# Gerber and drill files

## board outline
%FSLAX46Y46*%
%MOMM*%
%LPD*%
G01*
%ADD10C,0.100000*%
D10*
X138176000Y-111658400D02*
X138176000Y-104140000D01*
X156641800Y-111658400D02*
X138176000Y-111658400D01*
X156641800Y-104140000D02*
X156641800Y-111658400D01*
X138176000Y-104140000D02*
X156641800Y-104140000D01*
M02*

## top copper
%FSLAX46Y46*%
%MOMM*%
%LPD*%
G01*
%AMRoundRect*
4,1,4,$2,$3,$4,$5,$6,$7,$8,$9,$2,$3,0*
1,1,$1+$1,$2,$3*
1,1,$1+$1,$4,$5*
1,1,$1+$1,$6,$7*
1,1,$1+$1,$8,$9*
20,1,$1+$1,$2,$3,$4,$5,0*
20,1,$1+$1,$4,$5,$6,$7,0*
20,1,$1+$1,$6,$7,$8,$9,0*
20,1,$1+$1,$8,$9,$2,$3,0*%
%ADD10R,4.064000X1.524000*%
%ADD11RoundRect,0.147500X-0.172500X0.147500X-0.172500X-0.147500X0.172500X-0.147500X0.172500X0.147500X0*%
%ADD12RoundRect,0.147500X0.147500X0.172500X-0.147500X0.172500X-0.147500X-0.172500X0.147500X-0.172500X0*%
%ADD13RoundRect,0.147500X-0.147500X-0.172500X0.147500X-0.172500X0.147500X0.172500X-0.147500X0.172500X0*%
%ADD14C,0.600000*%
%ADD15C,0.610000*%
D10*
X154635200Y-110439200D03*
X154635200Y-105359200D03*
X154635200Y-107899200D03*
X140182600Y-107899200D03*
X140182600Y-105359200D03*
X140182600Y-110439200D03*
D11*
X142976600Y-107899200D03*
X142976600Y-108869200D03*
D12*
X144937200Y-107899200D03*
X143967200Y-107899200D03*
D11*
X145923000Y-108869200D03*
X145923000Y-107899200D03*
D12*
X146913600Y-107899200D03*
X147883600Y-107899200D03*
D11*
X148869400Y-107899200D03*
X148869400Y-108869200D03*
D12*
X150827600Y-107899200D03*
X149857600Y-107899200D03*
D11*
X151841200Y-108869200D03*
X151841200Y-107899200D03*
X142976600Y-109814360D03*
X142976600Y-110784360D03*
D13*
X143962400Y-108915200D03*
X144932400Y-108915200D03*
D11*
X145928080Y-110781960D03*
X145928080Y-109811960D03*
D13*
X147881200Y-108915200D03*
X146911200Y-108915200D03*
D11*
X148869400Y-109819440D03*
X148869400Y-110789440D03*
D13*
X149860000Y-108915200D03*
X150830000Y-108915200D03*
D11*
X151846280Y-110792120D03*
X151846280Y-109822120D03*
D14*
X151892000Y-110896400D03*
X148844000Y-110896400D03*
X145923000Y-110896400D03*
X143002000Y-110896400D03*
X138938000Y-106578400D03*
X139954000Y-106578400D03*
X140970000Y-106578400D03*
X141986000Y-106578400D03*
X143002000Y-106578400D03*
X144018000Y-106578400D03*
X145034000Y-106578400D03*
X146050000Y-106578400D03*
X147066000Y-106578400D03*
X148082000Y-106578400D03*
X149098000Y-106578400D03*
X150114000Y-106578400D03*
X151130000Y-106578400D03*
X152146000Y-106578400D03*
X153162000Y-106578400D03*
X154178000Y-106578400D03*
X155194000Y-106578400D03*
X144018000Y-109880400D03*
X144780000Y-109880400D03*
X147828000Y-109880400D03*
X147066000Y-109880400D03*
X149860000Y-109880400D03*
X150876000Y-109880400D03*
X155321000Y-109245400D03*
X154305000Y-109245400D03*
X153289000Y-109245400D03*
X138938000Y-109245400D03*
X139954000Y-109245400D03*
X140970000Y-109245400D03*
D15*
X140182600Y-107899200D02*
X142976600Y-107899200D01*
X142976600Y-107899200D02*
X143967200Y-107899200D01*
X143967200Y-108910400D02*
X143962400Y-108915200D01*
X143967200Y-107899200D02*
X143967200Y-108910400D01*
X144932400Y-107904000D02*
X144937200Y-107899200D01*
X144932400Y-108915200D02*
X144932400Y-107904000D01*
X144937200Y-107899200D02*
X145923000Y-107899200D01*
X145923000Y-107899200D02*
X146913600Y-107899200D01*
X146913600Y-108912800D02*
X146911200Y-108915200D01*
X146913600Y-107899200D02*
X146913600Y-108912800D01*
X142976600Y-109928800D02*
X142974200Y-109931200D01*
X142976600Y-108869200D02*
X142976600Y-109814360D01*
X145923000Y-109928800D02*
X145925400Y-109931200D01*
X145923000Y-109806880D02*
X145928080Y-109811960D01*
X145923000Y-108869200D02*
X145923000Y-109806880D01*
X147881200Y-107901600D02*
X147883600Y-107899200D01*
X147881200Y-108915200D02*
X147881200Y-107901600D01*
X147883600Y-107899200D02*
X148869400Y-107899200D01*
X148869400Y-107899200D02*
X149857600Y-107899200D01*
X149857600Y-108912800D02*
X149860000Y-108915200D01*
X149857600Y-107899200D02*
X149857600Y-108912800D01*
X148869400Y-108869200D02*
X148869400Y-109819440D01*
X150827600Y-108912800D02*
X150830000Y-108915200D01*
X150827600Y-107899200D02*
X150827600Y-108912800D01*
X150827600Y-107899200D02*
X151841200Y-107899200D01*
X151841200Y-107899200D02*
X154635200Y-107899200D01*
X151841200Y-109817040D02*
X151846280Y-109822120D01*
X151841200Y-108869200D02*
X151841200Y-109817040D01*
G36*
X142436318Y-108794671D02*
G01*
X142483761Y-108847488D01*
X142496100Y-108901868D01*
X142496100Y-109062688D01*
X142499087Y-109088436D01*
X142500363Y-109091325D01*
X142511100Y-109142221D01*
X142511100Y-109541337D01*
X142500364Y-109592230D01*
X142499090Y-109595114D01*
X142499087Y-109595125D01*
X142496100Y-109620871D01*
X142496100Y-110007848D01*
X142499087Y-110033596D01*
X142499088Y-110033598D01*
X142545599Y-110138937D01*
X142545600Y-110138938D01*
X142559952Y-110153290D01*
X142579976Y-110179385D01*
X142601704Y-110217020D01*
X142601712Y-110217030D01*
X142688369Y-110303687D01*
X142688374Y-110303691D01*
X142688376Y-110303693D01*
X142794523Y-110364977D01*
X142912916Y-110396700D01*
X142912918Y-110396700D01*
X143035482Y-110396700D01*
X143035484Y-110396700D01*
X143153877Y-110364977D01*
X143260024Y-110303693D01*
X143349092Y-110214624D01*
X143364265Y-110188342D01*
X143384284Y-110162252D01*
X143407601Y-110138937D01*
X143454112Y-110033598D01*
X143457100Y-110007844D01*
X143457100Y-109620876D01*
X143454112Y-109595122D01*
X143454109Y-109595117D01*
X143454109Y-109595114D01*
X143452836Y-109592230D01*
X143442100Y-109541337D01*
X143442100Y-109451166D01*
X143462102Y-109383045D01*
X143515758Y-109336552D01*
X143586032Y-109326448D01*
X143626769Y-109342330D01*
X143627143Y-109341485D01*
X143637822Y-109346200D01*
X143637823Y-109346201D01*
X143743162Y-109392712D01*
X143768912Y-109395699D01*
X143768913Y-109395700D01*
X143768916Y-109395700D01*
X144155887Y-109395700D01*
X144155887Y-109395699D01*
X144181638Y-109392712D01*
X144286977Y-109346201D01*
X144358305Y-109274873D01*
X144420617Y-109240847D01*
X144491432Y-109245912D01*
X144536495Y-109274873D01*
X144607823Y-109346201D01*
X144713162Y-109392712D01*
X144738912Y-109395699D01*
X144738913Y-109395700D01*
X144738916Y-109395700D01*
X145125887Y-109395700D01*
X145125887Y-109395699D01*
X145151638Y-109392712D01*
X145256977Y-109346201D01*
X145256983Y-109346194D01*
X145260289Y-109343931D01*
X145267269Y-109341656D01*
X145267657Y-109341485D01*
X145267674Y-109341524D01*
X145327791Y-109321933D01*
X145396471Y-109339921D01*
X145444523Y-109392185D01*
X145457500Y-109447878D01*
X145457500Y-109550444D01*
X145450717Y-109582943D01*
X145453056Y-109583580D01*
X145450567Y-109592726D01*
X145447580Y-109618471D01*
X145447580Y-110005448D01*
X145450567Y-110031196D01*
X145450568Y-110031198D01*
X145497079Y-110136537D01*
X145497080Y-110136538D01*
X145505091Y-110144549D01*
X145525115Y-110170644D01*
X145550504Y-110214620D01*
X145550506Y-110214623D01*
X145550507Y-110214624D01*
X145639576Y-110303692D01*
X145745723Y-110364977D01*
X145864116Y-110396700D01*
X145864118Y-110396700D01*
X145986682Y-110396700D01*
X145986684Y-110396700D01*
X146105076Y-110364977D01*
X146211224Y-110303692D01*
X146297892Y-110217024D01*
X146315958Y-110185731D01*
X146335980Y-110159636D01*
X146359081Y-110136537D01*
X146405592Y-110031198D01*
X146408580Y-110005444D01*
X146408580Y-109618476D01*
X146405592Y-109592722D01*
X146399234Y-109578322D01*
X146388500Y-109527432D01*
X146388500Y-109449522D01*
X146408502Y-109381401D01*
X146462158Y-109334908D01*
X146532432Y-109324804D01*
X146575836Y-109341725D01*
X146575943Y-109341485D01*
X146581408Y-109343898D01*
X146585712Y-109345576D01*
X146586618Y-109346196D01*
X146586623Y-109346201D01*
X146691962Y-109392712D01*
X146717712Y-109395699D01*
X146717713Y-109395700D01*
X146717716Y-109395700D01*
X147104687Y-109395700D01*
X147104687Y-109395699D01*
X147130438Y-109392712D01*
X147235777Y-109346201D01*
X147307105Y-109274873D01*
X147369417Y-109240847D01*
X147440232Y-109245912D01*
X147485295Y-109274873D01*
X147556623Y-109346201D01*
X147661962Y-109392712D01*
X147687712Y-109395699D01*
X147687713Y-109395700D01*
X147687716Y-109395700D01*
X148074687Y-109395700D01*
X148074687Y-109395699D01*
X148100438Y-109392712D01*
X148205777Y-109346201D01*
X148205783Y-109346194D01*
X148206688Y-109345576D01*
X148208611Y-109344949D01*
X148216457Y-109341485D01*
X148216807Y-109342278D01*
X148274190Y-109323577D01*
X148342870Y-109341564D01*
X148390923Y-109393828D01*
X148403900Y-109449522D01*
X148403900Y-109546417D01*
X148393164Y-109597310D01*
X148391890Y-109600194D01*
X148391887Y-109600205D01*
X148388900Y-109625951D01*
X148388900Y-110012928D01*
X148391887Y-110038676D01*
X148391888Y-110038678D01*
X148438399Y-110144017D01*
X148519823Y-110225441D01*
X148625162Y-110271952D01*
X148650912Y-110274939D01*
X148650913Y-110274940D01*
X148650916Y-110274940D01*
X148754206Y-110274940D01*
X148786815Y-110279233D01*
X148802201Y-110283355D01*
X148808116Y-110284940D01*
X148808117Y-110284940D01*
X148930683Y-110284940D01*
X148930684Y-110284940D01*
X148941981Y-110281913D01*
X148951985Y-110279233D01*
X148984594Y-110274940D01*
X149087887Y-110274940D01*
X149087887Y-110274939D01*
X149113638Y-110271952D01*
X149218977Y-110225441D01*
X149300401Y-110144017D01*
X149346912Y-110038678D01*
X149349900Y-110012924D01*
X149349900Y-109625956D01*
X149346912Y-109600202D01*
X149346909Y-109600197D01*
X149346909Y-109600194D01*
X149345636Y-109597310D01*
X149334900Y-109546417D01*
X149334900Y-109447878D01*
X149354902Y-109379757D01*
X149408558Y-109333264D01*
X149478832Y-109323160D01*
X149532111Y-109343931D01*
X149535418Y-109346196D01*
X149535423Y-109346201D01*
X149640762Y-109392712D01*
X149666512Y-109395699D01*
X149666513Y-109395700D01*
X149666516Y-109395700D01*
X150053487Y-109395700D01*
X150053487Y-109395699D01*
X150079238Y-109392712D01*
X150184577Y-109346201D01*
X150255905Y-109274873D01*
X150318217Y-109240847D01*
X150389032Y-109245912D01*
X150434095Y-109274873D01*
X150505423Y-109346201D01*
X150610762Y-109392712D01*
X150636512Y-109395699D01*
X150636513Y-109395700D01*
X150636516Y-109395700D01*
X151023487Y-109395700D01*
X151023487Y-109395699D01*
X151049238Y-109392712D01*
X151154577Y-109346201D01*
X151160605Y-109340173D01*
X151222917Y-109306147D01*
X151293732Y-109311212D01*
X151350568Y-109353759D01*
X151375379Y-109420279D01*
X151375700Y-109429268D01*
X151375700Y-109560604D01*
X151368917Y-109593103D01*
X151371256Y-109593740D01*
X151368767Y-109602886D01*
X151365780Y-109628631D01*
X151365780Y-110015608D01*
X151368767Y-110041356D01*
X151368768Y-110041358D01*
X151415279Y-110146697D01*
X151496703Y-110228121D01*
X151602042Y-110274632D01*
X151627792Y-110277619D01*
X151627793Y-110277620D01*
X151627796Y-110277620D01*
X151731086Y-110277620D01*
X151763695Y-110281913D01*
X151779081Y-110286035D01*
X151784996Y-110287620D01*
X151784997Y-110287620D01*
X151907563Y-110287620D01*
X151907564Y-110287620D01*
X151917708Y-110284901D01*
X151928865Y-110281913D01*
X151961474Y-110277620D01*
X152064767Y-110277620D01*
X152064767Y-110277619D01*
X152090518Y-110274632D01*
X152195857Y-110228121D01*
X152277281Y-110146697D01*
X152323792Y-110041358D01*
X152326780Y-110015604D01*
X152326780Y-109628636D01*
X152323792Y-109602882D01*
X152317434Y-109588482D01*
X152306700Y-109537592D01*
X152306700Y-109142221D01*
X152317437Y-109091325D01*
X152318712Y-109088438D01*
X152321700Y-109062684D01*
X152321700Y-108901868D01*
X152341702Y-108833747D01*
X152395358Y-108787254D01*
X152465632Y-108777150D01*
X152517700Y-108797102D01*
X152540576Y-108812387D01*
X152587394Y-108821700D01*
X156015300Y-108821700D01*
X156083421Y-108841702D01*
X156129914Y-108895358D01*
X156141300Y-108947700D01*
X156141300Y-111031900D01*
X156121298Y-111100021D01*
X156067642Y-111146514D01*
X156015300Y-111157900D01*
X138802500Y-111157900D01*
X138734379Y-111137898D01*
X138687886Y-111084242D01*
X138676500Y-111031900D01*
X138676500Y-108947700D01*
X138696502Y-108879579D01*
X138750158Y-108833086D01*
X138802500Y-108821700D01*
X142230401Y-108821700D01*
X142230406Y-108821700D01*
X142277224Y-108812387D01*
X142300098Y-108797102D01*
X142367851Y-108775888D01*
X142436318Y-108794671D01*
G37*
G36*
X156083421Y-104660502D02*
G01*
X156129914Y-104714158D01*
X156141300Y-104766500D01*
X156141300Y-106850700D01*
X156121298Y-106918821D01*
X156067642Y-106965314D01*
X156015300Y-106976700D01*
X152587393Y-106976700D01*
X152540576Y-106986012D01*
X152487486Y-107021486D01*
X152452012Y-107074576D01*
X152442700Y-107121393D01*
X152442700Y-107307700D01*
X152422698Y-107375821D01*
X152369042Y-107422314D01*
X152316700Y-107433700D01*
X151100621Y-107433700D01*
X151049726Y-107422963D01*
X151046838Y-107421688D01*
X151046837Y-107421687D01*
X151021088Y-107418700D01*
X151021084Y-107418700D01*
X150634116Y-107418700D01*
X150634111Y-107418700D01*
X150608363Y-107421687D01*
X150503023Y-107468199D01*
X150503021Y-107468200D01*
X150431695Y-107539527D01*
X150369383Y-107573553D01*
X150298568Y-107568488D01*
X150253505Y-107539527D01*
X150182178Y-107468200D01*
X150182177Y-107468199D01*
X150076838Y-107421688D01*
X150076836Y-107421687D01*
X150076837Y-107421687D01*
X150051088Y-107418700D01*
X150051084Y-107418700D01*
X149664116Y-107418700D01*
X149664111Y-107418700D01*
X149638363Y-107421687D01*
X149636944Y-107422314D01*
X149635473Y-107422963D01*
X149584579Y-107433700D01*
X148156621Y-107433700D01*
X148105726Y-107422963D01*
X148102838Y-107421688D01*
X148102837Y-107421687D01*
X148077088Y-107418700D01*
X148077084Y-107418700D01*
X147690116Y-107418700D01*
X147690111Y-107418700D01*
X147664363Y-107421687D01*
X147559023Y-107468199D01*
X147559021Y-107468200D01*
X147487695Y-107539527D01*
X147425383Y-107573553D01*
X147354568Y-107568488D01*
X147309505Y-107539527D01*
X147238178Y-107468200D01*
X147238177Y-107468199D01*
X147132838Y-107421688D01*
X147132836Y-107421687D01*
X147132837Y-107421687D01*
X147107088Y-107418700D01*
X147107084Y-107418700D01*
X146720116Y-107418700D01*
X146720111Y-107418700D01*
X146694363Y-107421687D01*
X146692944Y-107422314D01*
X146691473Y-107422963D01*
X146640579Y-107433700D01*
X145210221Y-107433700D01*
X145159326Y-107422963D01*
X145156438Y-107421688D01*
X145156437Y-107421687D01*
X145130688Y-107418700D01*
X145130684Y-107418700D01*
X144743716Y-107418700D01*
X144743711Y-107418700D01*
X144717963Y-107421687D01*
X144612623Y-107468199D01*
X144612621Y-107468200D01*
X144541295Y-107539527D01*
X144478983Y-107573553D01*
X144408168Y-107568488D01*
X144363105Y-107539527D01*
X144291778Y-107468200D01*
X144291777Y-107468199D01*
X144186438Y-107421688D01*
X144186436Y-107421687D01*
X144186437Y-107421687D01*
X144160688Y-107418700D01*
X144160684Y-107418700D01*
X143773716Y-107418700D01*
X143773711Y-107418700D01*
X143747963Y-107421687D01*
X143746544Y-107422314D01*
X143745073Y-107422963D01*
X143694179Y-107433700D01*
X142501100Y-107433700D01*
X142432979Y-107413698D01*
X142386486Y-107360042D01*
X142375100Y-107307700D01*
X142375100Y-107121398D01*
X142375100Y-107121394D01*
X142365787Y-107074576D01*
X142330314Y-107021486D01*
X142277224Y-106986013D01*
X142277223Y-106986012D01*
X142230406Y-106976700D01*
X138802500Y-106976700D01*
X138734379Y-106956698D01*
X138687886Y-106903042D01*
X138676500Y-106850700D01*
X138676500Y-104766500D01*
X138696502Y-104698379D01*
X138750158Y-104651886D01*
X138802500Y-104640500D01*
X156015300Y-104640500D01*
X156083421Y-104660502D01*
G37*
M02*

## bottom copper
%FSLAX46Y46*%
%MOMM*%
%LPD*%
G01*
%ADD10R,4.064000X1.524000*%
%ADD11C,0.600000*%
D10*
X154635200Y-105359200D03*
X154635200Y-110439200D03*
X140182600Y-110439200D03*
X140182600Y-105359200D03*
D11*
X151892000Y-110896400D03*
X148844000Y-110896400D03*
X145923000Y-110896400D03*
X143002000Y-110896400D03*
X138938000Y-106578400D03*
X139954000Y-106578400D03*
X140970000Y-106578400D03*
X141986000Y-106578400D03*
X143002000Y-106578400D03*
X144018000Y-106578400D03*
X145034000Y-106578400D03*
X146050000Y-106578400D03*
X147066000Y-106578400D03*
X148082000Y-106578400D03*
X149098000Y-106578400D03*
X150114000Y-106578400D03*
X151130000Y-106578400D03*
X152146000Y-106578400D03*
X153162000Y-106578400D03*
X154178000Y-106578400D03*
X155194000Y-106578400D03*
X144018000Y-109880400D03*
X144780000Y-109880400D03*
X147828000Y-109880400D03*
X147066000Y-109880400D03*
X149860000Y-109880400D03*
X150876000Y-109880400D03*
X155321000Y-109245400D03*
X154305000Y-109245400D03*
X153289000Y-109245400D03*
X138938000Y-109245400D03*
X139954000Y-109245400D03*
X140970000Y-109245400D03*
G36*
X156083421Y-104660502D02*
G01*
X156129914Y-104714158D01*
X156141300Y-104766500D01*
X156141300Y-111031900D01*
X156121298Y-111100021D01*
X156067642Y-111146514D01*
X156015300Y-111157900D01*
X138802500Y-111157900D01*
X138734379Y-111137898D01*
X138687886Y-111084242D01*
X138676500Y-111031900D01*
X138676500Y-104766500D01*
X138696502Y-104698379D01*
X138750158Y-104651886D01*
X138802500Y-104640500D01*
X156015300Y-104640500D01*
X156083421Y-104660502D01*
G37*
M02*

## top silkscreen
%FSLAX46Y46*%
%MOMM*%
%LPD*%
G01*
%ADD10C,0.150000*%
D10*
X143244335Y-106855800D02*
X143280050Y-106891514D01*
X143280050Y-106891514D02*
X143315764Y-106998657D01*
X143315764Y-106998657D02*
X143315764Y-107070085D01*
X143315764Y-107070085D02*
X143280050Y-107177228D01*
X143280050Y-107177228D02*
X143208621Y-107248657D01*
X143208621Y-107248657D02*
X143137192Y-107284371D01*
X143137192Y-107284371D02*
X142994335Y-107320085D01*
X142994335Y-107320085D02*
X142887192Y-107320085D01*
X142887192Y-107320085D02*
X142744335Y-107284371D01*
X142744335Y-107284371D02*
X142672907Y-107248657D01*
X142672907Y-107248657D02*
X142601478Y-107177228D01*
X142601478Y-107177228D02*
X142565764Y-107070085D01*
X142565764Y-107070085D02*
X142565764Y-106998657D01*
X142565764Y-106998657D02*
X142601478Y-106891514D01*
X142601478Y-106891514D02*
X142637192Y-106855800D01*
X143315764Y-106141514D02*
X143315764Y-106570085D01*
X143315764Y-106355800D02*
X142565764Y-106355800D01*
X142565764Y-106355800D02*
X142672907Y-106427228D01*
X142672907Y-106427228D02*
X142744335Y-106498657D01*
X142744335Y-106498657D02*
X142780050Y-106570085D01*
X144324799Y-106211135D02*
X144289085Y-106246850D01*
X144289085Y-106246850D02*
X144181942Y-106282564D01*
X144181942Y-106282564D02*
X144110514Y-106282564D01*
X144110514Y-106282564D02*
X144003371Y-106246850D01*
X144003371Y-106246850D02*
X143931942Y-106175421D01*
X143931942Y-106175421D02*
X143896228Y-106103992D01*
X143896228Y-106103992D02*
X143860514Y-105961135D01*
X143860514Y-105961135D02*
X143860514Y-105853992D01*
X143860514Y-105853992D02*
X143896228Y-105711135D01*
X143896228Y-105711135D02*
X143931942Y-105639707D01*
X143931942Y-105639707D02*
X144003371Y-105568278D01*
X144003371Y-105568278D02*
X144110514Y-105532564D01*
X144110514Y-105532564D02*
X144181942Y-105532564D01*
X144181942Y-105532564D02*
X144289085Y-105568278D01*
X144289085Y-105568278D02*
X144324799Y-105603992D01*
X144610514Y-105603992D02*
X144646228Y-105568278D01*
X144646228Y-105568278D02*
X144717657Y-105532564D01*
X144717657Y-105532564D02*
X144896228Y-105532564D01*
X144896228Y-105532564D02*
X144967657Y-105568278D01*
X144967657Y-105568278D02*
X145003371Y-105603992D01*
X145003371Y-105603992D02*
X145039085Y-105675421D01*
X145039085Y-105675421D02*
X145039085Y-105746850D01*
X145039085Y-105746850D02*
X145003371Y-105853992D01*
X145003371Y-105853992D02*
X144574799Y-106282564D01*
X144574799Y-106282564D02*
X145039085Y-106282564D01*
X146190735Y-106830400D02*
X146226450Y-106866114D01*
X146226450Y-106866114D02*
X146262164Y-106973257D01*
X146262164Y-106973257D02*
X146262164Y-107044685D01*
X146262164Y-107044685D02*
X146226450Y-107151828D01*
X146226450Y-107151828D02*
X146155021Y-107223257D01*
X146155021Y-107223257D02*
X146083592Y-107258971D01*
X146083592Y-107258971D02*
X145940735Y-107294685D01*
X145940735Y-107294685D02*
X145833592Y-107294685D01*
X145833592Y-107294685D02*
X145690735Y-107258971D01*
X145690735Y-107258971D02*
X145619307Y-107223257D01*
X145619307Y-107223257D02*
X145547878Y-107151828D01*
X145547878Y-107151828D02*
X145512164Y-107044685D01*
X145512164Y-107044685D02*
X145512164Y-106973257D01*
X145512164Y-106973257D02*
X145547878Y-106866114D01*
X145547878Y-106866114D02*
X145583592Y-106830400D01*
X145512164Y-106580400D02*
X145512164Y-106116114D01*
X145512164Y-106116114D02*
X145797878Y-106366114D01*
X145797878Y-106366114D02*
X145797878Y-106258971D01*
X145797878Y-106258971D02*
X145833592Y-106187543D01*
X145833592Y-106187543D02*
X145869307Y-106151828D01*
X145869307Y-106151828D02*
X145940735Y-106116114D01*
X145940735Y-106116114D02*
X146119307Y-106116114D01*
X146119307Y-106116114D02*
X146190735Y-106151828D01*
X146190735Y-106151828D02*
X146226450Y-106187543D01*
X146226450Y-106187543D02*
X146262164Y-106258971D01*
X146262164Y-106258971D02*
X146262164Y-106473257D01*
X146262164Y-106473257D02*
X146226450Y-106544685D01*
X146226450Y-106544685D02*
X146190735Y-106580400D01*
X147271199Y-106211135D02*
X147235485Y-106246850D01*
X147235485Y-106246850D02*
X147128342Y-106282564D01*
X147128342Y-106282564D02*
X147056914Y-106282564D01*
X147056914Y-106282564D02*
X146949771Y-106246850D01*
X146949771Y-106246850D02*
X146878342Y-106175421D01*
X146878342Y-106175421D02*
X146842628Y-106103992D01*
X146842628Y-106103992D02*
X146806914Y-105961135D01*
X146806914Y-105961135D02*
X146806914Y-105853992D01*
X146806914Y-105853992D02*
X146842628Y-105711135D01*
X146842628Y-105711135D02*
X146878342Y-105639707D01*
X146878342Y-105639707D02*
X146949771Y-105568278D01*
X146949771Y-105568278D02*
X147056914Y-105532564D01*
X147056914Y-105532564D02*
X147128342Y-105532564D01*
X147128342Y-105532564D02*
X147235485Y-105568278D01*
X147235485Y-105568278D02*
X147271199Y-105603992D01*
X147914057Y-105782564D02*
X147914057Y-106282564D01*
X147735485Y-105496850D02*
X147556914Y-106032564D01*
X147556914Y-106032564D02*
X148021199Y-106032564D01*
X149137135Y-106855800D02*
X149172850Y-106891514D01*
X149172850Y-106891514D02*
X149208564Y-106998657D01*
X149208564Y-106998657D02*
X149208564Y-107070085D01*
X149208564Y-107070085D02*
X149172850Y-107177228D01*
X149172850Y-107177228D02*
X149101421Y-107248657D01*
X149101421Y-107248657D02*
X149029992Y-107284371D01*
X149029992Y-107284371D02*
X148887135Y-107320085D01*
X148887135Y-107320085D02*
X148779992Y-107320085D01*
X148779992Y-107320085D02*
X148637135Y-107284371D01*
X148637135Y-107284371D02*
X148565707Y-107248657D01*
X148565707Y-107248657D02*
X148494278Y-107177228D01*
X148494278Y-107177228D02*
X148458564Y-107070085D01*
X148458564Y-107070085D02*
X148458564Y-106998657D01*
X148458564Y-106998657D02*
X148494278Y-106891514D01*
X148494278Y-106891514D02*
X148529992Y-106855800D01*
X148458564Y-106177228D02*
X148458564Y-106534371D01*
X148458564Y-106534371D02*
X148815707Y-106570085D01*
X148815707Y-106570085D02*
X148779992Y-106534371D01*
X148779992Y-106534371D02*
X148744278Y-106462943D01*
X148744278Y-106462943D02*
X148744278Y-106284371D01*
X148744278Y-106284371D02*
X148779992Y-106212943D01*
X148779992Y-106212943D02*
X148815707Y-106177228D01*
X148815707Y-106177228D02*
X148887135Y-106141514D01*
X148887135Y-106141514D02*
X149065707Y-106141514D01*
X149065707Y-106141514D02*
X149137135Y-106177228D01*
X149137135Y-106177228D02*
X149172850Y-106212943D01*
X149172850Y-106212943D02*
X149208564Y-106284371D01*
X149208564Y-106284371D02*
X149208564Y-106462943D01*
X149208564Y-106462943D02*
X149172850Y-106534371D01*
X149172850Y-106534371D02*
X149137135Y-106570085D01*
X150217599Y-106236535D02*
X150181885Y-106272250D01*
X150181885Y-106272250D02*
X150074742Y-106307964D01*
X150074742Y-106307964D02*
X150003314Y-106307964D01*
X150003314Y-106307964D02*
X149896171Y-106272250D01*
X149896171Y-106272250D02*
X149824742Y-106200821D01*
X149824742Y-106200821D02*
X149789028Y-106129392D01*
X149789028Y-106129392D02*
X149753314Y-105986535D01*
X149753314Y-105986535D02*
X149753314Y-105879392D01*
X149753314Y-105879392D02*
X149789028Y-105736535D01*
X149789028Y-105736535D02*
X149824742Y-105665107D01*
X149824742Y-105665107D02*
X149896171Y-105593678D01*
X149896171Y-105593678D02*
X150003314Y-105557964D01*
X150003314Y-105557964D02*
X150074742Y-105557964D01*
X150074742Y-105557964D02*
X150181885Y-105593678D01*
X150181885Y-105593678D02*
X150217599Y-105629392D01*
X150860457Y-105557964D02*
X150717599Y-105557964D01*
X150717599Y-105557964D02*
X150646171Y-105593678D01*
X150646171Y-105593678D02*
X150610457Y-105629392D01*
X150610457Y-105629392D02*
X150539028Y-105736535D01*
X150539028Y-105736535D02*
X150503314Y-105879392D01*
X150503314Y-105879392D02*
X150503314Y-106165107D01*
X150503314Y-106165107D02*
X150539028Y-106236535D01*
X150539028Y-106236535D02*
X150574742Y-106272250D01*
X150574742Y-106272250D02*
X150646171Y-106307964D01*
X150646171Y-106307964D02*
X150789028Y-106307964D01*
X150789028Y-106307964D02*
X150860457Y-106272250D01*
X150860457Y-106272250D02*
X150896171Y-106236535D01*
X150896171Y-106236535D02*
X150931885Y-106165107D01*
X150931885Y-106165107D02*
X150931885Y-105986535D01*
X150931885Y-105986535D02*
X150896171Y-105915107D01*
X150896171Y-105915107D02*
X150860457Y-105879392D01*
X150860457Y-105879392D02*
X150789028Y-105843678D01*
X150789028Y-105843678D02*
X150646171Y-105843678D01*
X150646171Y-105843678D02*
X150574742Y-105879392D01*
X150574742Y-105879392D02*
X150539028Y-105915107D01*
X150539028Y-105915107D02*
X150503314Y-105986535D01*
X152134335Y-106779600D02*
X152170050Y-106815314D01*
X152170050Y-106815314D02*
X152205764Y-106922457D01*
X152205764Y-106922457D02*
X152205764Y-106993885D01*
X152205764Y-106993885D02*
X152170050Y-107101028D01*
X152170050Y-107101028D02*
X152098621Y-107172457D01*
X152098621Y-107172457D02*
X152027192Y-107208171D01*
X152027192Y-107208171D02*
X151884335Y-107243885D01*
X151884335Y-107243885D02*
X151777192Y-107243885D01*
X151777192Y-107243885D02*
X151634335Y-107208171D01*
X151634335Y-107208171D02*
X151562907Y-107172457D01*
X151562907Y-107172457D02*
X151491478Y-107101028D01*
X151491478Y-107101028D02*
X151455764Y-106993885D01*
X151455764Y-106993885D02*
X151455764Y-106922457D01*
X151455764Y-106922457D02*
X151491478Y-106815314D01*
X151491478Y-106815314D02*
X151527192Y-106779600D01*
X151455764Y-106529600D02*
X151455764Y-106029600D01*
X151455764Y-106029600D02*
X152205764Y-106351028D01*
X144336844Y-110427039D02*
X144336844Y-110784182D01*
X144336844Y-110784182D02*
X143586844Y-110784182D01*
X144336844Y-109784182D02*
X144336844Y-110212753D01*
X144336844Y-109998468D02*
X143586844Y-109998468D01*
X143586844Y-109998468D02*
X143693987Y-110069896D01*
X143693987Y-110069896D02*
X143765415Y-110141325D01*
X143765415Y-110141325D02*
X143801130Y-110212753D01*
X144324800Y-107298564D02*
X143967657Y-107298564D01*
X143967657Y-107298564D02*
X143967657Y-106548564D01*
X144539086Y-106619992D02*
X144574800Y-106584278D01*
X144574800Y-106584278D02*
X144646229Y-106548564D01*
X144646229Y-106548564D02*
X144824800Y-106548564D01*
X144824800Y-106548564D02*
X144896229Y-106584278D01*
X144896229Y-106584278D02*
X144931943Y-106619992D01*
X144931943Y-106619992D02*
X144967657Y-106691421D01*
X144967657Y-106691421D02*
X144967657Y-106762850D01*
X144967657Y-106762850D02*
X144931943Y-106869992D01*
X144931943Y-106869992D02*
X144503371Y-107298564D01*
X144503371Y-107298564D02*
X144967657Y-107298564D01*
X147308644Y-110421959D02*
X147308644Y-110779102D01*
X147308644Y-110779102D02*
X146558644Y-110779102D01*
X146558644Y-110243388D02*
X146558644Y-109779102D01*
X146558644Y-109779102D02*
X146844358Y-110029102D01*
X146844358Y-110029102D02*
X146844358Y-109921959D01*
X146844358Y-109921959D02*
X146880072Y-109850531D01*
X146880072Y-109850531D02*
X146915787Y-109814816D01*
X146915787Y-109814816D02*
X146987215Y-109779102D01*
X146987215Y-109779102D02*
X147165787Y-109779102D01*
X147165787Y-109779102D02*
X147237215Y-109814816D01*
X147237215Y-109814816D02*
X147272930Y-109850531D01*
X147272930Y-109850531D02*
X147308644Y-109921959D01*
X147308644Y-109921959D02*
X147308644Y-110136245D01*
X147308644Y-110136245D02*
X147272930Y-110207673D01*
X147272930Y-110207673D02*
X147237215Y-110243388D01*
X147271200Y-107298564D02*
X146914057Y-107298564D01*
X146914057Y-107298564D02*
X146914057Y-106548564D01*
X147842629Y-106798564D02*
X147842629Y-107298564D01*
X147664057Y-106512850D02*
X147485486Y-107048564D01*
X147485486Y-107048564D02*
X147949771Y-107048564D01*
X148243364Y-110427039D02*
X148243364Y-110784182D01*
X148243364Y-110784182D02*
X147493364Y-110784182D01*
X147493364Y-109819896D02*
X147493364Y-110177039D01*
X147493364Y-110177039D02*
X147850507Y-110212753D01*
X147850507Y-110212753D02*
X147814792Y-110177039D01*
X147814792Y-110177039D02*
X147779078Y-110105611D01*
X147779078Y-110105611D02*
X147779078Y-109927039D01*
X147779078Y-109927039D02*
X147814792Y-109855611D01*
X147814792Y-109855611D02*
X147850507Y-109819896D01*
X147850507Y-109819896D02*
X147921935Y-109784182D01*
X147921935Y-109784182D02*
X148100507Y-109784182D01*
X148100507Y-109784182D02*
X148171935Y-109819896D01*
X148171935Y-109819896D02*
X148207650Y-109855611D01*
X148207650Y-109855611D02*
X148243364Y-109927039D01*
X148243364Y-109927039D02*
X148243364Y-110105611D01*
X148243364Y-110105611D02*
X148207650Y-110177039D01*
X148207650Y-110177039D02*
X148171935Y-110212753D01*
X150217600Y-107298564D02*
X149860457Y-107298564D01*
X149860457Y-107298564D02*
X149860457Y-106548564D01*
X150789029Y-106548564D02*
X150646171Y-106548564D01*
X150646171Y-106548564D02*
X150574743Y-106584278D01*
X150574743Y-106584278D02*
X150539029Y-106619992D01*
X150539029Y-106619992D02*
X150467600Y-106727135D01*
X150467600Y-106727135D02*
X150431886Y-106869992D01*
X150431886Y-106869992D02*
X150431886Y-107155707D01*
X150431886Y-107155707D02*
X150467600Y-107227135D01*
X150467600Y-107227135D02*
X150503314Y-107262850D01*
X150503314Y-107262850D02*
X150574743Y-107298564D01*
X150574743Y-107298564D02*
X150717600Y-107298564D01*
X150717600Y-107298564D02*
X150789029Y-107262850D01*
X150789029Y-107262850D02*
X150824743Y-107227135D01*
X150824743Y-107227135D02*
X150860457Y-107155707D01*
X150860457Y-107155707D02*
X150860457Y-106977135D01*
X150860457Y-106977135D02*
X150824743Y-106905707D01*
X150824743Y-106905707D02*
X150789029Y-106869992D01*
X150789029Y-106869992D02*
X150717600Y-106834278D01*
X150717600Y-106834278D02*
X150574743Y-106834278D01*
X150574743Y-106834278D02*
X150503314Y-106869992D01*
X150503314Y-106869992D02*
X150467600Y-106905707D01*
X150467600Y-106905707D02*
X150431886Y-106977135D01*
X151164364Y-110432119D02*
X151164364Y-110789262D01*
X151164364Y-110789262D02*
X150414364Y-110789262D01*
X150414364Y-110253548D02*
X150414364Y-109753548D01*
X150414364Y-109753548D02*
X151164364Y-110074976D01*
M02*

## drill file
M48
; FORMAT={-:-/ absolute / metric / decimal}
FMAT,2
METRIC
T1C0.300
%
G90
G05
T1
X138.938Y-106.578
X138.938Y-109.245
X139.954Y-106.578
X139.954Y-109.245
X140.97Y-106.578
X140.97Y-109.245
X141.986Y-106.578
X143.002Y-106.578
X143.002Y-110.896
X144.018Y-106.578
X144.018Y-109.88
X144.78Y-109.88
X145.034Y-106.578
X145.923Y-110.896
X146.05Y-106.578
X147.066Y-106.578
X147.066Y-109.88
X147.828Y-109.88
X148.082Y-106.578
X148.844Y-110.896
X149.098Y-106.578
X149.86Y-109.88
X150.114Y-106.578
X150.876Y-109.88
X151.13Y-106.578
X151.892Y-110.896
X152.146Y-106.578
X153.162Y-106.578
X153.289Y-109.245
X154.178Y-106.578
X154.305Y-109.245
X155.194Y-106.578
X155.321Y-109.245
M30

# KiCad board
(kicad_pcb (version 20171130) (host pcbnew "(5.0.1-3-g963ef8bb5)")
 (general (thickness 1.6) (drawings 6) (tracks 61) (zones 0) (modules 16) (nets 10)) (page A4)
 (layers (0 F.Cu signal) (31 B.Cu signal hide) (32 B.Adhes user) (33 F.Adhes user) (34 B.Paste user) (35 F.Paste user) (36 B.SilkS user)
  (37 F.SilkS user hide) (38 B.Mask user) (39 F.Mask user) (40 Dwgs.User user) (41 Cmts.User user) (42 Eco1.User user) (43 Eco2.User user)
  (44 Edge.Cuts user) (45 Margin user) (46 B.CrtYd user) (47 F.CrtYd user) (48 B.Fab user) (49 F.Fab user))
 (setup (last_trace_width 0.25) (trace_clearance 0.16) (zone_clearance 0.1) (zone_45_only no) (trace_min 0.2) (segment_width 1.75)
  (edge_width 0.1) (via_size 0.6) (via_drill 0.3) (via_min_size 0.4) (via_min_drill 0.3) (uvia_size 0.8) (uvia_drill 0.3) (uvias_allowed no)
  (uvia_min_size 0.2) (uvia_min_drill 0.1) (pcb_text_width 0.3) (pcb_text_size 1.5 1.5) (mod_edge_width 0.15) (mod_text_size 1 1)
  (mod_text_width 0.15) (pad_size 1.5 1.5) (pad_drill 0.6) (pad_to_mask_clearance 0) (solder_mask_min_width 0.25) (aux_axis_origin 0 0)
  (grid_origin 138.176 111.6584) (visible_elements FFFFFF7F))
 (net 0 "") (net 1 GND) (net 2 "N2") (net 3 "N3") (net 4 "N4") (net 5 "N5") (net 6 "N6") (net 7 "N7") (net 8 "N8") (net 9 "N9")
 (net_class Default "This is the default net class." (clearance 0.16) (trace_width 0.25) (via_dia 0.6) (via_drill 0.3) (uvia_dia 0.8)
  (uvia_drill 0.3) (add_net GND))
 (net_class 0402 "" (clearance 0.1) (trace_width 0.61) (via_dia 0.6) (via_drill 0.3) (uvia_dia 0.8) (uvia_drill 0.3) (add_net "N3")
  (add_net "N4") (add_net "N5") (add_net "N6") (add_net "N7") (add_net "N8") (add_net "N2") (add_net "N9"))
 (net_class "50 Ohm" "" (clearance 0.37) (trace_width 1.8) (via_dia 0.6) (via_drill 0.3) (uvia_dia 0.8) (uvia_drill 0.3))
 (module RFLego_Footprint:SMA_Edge (layer F.Cu) (at 152.6032 107.8992)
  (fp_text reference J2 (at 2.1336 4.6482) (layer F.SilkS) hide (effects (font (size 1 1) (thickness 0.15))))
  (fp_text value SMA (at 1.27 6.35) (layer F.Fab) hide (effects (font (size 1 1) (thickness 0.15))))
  (pad 2 smd rect (at 2.032 2.54) (size 4.064 1.524) (layers F.Cu F.Mask) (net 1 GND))
  (pad 2 smd rect (at 2.032 -2.54) (size 4.064 1.524) (layers B.Cu B.Mask) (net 1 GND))
  (pad 2 smd rect (at 2.032 2.54) (size 4.064 1.524) (layers B.Cu B.Mask) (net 1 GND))
  (pad 2 smd rect (at 2.032 -2.54) (size 4.064 1.524) (layers F.Cu F.Mask) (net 1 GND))
  (pad 1 smd rect (at 2.032 0) (size 4.064 1.524) (layers F.Cu F.Mask) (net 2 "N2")))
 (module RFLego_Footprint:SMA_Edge (layer F.Cu) (at 138.1506 107.8992)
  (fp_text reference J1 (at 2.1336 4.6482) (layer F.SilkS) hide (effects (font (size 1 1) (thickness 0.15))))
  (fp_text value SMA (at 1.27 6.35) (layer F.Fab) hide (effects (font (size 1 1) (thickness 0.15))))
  (pad 1 smd rect (at 2.032 0) (size 4.064 1.524) (layers F.Cu F.Mask) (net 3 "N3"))
  (pad 2 smd rect (at 2.032 -2.54) (size 4.064 1.524) (layers F.Cu F.Mask) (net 1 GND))
  (pad 2 smd rect (at 2.032 2.54) (size 4.064 1.524) (layers B.Cu B.Mask) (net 1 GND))
  (pad 2 smd rect (at 2.032 -2.54) (size 4.064 1.524) (layers B.Cu B.Mask) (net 1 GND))
  (pad 2 smd rect (at 2.032 2.54) (size 4.064 1.524) (layers F.Cu F.Mask) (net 1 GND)))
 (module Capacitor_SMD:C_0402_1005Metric (layer F.Cu) (at 142.9766 108.3842 270)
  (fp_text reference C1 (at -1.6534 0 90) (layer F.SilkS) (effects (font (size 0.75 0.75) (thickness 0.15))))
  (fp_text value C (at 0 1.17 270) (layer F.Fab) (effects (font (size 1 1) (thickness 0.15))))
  (pad 1 smd roundrect (at -0.485 0 270) (size 0.59 0.64) (layers F.Cu F.Paste F.Mask) (roundrect_rratio 0.25) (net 3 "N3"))
  (pad 2 smd roundrect (at 0.485 0 270) (size 0.59 0.64) (layers F.Cu F.Paste F.Mask) (roundrect_rratio 0.25) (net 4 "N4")))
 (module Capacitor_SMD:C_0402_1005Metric (layer F.Cu) (at 144.4522 107.8992 180)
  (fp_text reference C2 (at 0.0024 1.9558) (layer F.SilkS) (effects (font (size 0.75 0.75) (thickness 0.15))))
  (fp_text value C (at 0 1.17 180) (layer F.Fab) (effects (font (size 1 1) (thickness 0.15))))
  (pad 1 smd roundrect (at -0.485 0 180) (size 0.59 0.64) (layers F.Cu F.Paste F.Mask) (roundrect_rratio 0.25) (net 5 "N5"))
  (pad 2 smd roundrect (at 0.485 0 180) (size 0.59 0.64) (layers F.Cu F.Paste F.Mask) (roundrect_rratio 0.25) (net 3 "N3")))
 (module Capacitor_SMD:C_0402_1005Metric (layer F.Cu) (at 145.923 108.3842 270)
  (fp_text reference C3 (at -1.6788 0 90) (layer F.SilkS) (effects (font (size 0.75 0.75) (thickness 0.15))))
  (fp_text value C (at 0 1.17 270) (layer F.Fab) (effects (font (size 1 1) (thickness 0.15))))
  (pad 2 smd roundrect (at 0.485 0 270) (size 0.59 0.64) (layers F.Cu F.Paste F.Mask) (roundrect_rratio 0.25) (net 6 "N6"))
  (pad 1 smd roundrect (at -0.485 0 270) (size 0.59 0.64) (layers F.Cu F.Paste F.Mask) (roundrect_rratio 0.25) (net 5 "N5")))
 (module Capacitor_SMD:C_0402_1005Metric (layer F.Cu) (at 147.3986 107.8992 180)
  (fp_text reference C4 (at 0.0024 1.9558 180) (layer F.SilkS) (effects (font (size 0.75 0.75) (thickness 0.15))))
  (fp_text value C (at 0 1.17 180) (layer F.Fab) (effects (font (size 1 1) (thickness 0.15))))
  (pad 2 smd roundrect (at 0.485 0 180) (size 0.59 0.64) (layers F.Cu F.Paste F.Mask) (roundrect_rratio 0.25) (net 5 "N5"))
  (pad 1 smd roundrect (at -0.485 0 180) (size 0.59 0.64) (layers F.Cu F.Paste F.Mask) (roundrect_rratio 0.25) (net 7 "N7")))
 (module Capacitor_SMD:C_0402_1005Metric (layer F.Cu) (at 148.8694 108.3842 270)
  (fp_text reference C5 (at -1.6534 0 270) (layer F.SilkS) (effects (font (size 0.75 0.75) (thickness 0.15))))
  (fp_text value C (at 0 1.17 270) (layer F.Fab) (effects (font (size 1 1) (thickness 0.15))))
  (pad 1 smd roundrect (at -0.485 0 270) (size 0.59 0.64) (layers F.Cu F.Paste F.Mask) (roundrect_rratio 0.25) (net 7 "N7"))
  (pad 2 smd roundrect (at 0.485 0 270) (size 0.59 0.64) (layers F.Cu F.Paste F.Mask) (roundrect_rratio 0.25) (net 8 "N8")))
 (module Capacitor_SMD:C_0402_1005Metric (layer F.Cu) (at 150.3426 107.8992 180)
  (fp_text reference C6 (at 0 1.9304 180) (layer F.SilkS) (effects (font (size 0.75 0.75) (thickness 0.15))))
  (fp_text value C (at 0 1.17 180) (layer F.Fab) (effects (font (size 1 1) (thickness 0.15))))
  (pad 1 smd roundrect (at -0.485 0 180) (size 0.59 0.64) (layers F.Cu F.Paste F.Mask) (roundrect_rratio 0.25) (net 2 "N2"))
  (pad 2 smd roundrect (at 0.485 0 180) (size 0.59 0.64) (layers F.Cu F.Paste F.Mask) (roundrect_rratio 0.25) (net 7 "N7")))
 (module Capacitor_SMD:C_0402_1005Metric (layer F.Cu) (at 151.8412 108.3842 270)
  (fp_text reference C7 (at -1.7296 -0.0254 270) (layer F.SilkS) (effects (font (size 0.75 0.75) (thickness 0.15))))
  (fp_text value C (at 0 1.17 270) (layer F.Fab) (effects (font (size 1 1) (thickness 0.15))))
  (pad 2 smd roundrect (at 0.485 0 270) (size 0.59 0.64) (layers F.Cu F.Paste F.Mask) (roundrect_rratio 0.25) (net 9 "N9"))
  (pad 1 smd roundrect (at -0.485 0 270) (size 0.59 0.64) (layers F.Cu F.Paste F.Mask) (roundrect_rratio 0.25) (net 2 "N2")))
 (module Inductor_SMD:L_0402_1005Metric (layer F.Cu) (at 142.9766 110.29936 270)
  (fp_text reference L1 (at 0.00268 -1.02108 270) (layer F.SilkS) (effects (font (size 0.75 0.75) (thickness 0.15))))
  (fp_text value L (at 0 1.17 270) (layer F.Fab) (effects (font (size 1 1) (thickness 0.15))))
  (pad 1 smd roundrect (at -0.485 0 270) (size 0.59 0.64) (layers F.Cu F.Paste F.Mask) (roundrect_rratio 0.25) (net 4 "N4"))
  (pad 2 smd roundrect (at 0.485 0 270) (size 0.59 0.64) (layers F.Cu F.Paste F.Mask) (roundrect_rratio 0.25) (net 1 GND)))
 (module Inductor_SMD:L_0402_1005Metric (layer F.Cu) (at 144.4474 108.9152)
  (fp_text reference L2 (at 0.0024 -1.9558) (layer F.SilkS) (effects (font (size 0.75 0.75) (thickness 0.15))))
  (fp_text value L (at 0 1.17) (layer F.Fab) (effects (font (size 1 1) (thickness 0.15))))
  (pad 1 smd roundrect (at -0.485 0) (size 0.59 0.64) (layers F.Cu F.Paste F.Mask) (roundrect_rratio 0.25) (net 3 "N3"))
  (pad 2 smd roundrect (at 0.485 0) (size 0.59 0.64) (layers F.Cu F.Paste F.Mask) (roundrect_rratio 0.25) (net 5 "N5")))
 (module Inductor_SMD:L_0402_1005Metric (layer F.Cu) (at 145.92808 110.29696 270)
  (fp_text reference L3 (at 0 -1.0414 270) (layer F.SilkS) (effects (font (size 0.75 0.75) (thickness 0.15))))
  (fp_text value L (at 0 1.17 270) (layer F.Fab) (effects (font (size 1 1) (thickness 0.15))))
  (pad 2 smd roundrect (at 0.485 0 270) (size 0.59 0.64) (layers F.Cu F.Paste F.Mask) (roundrect_rratio 0.25) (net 1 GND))
  (pad 1 smd roundrect (at -0.485 0 270) (size 0.59 0.64) (layers F.Cu F.Paste F.Mask) (roundrect_rratio 0.25) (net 6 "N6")))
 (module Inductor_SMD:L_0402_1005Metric (layer F.Cu) (at 147.3962 108.9152)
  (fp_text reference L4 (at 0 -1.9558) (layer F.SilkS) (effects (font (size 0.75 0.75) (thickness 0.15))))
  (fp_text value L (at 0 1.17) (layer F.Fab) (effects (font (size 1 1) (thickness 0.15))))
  (pad 2 smd roundrect (at 0.485 0) (size 0.59 0.64) (layers F.Cu F.Paste F.Mask) (roundrect_rratio 0.25) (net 7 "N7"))
  (pad 1 smd roundrect (at -0.485 0) (size 0.59 0.64) (layers F.Cu F.Paste F.Mask) (roundrect_rratio 0.25) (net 5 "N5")))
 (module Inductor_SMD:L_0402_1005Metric (layer F.Cu) (at 148.8694 110.30444 270)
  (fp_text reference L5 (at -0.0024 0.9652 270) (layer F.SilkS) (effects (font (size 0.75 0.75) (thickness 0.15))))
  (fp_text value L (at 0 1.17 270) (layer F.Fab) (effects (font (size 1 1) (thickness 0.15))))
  (pad 1 smd roundrect (at -0.485 0 270) (size 0.59 0.64) (layers F.Cu F.Paste F.Mask) (roundrect_rratio 0.25) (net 8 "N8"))
  (pad 2 smd roundrect (at 0.485 0 270) (size 0.59 0.64) (layers F.Cu F.Paste F.Mask) (roundrect_rratio 0.25) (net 1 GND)))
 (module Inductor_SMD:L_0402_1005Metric (layer F.Cu) (at 150.345 108.9152)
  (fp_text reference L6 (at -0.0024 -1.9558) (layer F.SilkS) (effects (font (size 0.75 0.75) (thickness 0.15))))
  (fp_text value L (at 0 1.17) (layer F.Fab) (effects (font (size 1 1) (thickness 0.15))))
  (pad 1 smd roundrect (at -0.485 0) (size 0.59 0.64) (layers F.Cu F.Paste F.Mask) (roundrect_rratio 0.25) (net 7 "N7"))
  (pad 2 smd roundrect (at 0.485 0) (size 0.59 0.64) (layers F.Cu F.Paste F.Mask) (roundrect_rratio 0.25) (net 2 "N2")))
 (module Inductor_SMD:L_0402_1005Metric (layer F.Cu) (at 151.84628 110.30712 270)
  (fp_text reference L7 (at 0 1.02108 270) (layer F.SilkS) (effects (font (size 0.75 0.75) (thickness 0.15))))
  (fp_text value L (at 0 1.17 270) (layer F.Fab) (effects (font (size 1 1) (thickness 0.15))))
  (pad 2 smd roundrect (at 0.485 0 270) (size 0.59 0.64) (layers F.Cu F.Paste F.Mask) (roundrect_rratio 0.25) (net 1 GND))
  (pad 1 smd roundrect (at -0.485 0 270) (size 0.59 0.64) (layers F.Cu F.Paste F.Mask) (roundrect_rratio 0.25) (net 9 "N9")))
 (gr_line (start 138.176 111.6584) (end 138.176 104.14) (layer Edge.Cuts) (width 0.1))
 (gr_line (start 156.6418 111.6584) (end 138.176 111.6584) (layer Edge.Cuts) (width 0.1))
 (gr_line (start 156.6418 104.14) (end 156.6418 111.6584) (layer Edge.Cuts) (width 0.1))
 (gr_line (start 138.176 104.14) (end 156.6418 104.14) (layer Edge.Cuts) (width 0.1))
 (segment (start 140.1826 107.8992) (end 142.9766 107.8992) (width 0.61) (layer F.Cu) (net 3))
 (segment (start 142.9766 107.8992) (end 143.9672 107.8992) (width 0.61) (layer F.Cu) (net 3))
 (segment (start 143.9672 108.9104) (end 143.9624 108.9152) (width 0.61) (layer F.Cu) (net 3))
 (segment (start 143.9672 107.8992) (end 143.9672 108.9104) (width 0.61) (layer F.Cu) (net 3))
 (via (at 151.892 110.8964) (size 0.6) (drill 0.3) (layers F.Cu B.Cu) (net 1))
 (via (at 148.844 110.8964) (size 0.6) (drill 0.3) (layers F.Cu B.Cu) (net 1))
 (via (at 145.923 110.8964) (size 0.6) (drill 0.3) (layers F.Cu B.Cu) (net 1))
 (via (at 143.002 110.8964) (size 0.6) (drill 0.3) (layers F.Cu B.Cu) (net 1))
 (via (at 138.938 106.5784) (size 0.6) (drill 0.3) (layers F.Cu B.Cu) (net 1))
 (via (at 139.954 106.5784) (size 0.6) (drill 0.3) (layers F.Cu B.Cu) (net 1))
 (via (at 140.97 106.5784) (size 0.6) (drill 0.3) (layers F.Cu B.Cu) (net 1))
 (via (at 141.986 106.5784) (size 0.6) (drill 0.3) (layers F.Cu B.Cu) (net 1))
 (via (at 143.002 106.5784) (size 0.6) (drill 0.3) (layers F.Cu B.Cu) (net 1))
 (via (at 144.018 106.5784) (size 0.6) (drill 0.3) (layers F.Cu B.Cu) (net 1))
 (via (at 145.034 106.5784) (size 0.6) (drill 0.3) (layers F.Cu B.Cu) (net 1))
 (via (at 146.05 106.5784) (size 0.6) (drill 0.3) (layers F.Cu B.Cu) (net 1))
 (via (at 147.066 106.5784) (size 0.6) (drill 0.3) (layers F.Cu B.Cu) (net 1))
 (via (at 148.082 106.5784) (size 0.6) (drill 0.3) (layers F.Cu B.Cu) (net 1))
 (via (at 149.098 106.5784) (size 0.6) (drill 0.3) (layers F.Cu B.Cu) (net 1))
 (via (at 150.114 106.5784) (size 0.6) (drill 0.3) (layers F.Cu B.Cu) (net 1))
 (via (at 151.13 106.5784) (size 0.6) (drill 0.3) (layers F.Cu B.Cu) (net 1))
 (via (at 152.146 106.5784) (size 0.6) (drill 0.3) (layers F.Cu B.Cu) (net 1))
 (via (at 153.162 106.5784) (size 0.6) (drill 0.3) (layers F.Cu B.Cu) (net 1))
 (via (at 154.178 106.5784) (size 0.6) (drill 0.3) (layers F.Cu B.Cu) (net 1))
 (via (at 155.194 106.5784) (size 0.6) (drill 0.3) (layers F.Cu B.Cu) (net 1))
 (via (at 144.018 109.8804) (size 0.6) (drill 0.3) (layers F.Cu B.Cu) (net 1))
 (via (at 144.78 109.8804) (size 0.6) (drill 0.3) (layers F.Cu B.Cu) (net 1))
 (via (at 147.828 109.8804) (size 0.6) (drill 0.3) (layers F.Cu B.Cu) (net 1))
 (via (at 147.066 109.8804) (size 0.6) (drill 0.3) (layers F.Cu B.Cu) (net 1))
 (via (at 149.86 109.8804) (size 0.6) (drill 0.3) (layers F.Cu B.Cu) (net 1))
 (via (at 150.876 109.8804) (size 0.6) (drill 0.3) (layers F.Cu B.Cu) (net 1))
 (via (at 155.321 109.2454) (size 0.6) (drill 0.3) (layers F.Cu B.Cu) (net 1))
 (via (at 154.305 109.2454) (size 0.6) (drill 0.3) (layers F.Cu B.Cu) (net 1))
 (via (at 153.289 109.2454) (size 0.6) (drill 0.3) (layers F.Cu B.Cu) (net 1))
 (via (at 138.938 109.2454) (size 0.6) (drill 0.3) (layers F.Cu B.Cu) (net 1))
 (via (at 139.954 109.2454) (size 0.6) (drill 0.3) (layers F.Cu B.Cu) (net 1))
 (via (at 140.97 109.2454) (size 0.6) (drill 0.3) (layers F.Cu B.Cu) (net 1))
 (segment (start 144.9324 107.904) (end 144.9372 107.8992) (width 0.61) (layer F.Cu) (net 5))
 (segment (start 144.9324 108.9152) (end 144.9324 107.904) (width 0.61) (layer F.Cu) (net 5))
 (segment (start 144.9372 107.8992) (end 145.923 107.8992) (width 0.61) (layer F.Cu) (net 5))
 (segment (start 145.923 107.8992) (end 146.9136 107.8992) (width 0.61) (layer F.Cu) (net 5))
 (segment (start 146.9136 108.9128) (end 146.9112 108.9152) (width 0.61) (layer F.Cu) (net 5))
 (segment (start 146.9136 107.8992) (end 146.9136 108.9128) (width 0.61) (layer F.Cu) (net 5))
 (segment (start 142.9766 109.9288) (end 142.9742 109.9312) (width 0.61) (layer F.Cu) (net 4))
 (segment (start 142.9766 108.8692) (end 142.9766 109.81436) (width 0.61) (layer F.Cu) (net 4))
 (segment (start 145.923 109.9288) (end 145.9254 109.9312) (width 0.61) (layer F.Cu) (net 6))
 (segment (start 145.923 109.80688) (end 145.92808 109.81196) (width 0.61) (layer F.Cu) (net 6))
 (segment (start 145.923 108.8692) (end 145.923 109.80688) (width 0.61) (layer F.Cu) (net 6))
 (segment (start 147.8812 107.9016) (end 147.8836 107.8992) (width 0.61) (layer F.Cu) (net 7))
 (segment (start 147.8812 108.9152) (end 147.8812 107.9016) (width 0.61) (layer F.Cu) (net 7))
 (segment (start 147.8836 107.8992) (end 148.8694 107.8992) (width 0.61) (layer F.Cu) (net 7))
 (segment (start 148.8694 107.8992) (end 149.8576 107.8992) (width 0.61) (layer F.Cu) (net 7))
 (segment (start 149.8576 108.9128) (end 149.86 108.9152) (width 0.61) (layer F.Cu) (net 7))
 (segment (start 149.8576 107.8992) (end 149.8576 108.9128) (width 0.61) (layer F.Cu) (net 7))
 (segment (start 148.8694 108.8692) (end 148.8694 109.81944) (width 0.61) (layer F.Cu) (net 8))
 (segment (start 150.8276 108.9128) (end 150.83 108.9152) (width 0.61) (layer F.Cu) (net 2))
 (segment (start 150.8276 107.8992) (end 150.8276 108.9128) (width 0.61) (layer F.Cu) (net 2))
 (segment (start 150.8276 107.8992) (end 151.8412 107.8992) (width 0.61) (layer F.Cu) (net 2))
 (segment (start 151.8412 107.8992) (end 154.6352 107.8992) (width 0.61) (layer F.Cu) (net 2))
 (segment (start 151.8412 109.81704) (end 151.84628 109.82212) (width 0.61) (layer F.Cu) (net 9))
 (segment (start 151.8412 108.8692) (end 151.8412 109.81704) (width 0.61) (layer F.Cu) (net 9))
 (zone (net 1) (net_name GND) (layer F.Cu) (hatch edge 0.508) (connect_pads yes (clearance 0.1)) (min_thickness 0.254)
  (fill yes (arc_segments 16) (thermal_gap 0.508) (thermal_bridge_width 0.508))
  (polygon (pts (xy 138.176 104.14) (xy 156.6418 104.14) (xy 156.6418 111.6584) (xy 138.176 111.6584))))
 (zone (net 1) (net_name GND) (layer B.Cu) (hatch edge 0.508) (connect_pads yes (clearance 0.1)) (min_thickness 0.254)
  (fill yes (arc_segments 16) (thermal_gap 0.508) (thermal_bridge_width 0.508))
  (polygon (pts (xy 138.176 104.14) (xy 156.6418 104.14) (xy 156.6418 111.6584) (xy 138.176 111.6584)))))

